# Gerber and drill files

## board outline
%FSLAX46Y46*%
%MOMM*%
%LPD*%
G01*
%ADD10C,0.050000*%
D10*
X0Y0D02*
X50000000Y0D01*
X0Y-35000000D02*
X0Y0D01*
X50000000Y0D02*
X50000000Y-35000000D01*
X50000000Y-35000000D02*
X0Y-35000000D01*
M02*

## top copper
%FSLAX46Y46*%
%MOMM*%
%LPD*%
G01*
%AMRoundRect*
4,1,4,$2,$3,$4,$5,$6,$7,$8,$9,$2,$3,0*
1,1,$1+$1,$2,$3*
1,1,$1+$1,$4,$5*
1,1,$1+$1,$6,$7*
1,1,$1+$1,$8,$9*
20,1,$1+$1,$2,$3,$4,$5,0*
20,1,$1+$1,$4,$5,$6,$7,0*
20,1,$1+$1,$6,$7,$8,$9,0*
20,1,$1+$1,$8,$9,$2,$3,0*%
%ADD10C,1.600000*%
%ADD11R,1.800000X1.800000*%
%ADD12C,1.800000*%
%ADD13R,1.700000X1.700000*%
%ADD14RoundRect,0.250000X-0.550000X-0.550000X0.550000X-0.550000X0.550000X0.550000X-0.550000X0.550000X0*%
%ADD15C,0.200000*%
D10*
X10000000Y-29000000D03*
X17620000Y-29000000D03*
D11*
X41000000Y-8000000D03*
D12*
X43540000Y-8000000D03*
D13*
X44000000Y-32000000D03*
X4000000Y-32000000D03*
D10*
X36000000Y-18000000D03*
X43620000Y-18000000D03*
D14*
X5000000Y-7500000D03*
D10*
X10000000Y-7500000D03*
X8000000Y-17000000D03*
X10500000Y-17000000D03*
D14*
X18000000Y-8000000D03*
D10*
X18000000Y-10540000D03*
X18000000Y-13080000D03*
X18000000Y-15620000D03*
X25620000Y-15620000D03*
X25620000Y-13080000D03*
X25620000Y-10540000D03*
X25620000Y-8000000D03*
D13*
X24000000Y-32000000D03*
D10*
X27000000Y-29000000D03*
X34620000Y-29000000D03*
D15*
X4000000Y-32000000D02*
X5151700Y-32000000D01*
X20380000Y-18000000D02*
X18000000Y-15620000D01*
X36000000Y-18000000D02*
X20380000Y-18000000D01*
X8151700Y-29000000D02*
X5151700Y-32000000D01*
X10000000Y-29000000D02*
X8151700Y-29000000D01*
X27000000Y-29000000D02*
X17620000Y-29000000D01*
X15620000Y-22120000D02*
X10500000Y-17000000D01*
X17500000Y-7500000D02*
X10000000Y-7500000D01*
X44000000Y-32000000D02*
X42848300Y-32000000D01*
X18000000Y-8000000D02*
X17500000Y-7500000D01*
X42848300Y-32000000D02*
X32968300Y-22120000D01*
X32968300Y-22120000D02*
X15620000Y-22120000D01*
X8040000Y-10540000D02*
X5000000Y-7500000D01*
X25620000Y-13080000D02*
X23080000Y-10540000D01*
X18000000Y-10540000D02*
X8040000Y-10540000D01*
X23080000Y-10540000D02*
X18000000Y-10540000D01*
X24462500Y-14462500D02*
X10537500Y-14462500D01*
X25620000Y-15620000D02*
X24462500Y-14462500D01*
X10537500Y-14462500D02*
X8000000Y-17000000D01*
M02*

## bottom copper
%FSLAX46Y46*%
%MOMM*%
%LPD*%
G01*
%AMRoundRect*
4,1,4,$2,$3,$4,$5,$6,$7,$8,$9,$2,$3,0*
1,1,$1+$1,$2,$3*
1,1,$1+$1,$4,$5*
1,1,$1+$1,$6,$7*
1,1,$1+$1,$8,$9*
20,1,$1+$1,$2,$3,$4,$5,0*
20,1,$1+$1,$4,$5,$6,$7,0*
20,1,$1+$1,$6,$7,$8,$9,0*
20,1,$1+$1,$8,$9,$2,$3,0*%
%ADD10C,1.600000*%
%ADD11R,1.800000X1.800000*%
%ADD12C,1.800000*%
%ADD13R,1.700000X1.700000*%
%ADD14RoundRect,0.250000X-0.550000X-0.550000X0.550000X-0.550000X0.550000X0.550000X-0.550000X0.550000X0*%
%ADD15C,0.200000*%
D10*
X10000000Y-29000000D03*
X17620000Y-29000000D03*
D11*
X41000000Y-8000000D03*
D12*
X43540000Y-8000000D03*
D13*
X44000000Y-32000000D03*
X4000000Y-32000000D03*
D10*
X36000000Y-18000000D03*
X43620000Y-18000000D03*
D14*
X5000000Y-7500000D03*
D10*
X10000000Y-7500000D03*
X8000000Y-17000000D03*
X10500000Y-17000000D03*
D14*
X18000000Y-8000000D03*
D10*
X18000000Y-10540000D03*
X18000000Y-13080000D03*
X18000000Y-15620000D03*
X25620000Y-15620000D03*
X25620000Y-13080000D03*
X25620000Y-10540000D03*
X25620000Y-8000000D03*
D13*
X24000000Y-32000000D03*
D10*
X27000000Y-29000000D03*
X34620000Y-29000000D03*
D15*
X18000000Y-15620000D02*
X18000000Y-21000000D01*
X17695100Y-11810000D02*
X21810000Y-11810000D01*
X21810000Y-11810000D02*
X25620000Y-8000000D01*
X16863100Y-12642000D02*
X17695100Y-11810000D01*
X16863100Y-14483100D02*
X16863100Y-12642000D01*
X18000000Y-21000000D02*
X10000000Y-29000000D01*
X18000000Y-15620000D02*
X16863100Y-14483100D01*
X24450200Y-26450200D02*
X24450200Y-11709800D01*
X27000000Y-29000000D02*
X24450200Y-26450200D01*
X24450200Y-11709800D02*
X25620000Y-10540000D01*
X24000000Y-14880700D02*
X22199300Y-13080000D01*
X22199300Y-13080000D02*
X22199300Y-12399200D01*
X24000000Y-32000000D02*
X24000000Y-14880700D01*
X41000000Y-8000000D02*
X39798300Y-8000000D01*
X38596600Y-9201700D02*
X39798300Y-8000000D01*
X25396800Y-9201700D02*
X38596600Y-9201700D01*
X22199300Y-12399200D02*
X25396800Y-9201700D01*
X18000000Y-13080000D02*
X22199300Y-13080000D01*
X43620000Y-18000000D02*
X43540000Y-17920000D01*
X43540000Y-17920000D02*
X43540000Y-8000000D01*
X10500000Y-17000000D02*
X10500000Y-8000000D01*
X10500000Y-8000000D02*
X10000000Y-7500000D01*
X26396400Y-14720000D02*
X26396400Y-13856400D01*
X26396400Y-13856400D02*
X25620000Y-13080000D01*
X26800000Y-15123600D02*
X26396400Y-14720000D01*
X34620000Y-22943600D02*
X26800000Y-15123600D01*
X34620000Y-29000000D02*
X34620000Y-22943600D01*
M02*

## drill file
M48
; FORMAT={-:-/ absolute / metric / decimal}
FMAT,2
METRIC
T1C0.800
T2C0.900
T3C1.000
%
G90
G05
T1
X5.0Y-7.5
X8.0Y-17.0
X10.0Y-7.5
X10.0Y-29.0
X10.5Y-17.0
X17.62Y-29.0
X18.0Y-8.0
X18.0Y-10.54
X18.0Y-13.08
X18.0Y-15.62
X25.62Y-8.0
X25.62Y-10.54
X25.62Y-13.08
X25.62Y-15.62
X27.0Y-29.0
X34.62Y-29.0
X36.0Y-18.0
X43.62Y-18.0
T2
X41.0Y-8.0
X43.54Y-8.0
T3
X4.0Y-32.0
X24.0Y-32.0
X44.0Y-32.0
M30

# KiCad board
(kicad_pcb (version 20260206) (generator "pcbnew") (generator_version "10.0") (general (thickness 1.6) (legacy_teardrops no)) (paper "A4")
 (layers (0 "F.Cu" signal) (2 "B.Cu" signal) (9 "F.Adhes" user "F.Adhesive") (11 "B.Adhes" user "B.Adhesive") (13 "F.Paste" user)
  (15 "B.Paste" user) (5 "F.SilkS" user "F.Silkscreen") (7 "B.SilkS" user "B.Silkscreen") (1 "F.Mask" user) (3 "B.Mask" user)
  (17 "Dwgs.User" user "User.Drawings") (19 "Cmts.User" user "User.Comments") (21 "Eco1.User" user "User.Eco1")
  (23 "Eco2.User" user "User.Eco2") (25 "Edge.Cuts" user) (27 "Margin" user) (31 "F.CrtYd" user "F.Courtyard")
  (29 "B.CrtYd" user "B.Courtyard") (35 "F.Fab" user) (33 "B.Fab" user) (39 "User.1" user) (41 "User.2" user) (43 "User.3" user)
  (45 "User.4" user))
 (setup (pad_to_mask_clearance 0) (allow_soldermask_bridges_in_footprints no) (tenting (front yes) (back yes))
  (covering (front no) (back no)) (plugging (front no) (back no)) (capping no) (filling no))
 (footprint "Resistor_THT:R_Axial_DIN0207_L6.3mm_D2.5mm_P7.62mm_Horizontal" (layer "F.Cu") (at 10 29)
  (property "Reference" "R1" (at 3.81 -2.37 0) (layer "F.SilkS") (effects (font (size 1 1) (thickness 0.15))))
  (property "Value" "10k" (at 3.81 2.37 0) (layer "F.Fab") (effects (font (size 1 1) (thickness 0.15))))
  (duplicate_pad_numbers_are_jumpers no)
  (pad "1" thru_hole circle (at 0 0) (size 1.6 1.6) (drill 0.8) (layers "*.Cu" "*.Mask") (remove_unused_layers no) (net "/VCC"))
  (pad "2" thru_hole circle (at 7.62 0) (size 1.6 1.6) (drill 0.8) (layers "*.Cu" "*.Mask") (remove_unused_layers no) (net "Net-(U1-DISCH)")))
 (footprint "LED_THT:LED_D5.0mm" (layer "F.Cu") (at 41 8)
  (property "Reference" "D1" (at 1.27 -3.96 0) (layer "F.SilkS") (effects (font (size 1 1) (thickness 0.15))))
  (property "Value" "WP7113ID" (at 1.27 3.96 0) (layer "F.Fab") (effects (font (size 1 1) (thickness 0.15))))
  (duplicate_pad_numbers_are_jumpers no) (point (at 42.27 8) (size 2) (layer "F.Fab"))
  (pad "1" thru_hole rect (at 0 0) (size 1.8 1.8) (drill 0.9) (layers "*.Cu" "*.Mask") (remove_unused_layers no) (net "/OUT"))
  (pad "2" thru_hole circle (at 2.54 0) (size 1.8 1.8) (drill 0.9) (layers "*.Cu" "*.Mask") (remove_unused_layers no) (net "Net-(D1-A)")))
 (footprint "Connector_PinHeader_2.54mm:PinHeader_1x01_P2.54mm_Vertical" (layer "F.Cu") (at 44 32)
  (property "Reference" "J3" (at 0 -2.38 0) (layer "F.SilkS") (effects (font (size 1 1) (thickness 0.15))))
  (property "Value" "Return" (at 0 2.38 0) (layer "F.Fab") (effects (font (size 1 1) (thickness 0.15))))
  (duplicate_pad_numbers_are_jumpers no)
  (pad "1" thru_hole rect (at 0 0) (size 1.7 1.7) (drill 1) (layers "*.Cu" "*.Mask") (remove_unused_layers no) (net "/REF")))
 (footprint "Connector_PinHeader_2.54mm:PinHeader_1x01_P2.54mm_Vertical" (layer "F.Cu") (at 4 32)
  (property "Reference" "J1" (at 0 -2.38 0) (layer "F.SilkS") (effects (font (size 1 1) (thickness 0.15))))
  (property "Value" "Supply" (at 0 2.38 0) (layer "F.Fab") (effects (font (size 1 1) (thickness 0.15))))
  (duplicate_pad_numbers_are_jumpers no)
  (pad "1" thru_hole rect (at 0 0) (size 1.7 1.7) (drill 1) (layers "*.Cu" "*.Mask") (remove_unused_layers no) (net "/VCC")))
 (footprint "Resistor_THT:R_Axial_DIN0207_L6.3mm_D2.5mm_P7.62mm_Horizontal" (layer "F.Cu") (at 36 18)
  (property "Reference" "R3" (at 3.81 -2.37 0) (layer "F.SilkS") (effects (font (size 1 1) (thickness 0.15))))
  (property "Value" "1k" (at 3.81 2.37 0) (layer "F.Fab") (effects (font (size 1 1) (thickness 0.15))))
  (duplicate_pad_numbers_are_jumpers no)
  (pad "1" thru_hole circle (at 0 0) (size 1.6 1.6) (drill 0.8) (layers "*.Cu" "*.Mask") (remove_unused_layers no) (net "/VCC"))
  (pad "2" thru_hole circle (at 7.62 0) (size 1.6 1.6) (drill 0.8) (layers "*.Cu" "*.Mask") (remove_unused_layers no) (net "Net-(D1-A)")))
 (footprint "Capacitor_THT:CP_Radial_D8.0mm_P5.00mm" (layer "F.Cu") (at 5 7.5)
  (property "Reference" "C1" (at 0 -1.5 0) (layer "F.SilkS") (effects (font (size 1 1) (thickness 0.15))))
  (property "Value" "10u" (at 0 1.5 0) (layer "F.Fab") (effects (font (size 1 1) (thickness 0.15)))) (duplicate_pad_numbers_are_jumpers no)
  (pad "1" thru_hole roundrect (at 0 0) (size 1.6 1.6) (drill 0.8) (layers "*.Cu" "*.Mask") (remove_unused_layers no)
   (roundrect_rratio 0.15625) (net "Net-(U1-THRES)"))
  (pad "2" thru_hole circle (at 5 0) (size 1.6 1.6) (drill 0.8) (layers "*.Cu" "*.Mask") (remove_unused_layers no) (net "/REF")))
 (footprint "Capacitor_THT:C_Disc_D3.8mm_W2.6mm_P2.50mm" (layer "F.Cu") (at 8 17)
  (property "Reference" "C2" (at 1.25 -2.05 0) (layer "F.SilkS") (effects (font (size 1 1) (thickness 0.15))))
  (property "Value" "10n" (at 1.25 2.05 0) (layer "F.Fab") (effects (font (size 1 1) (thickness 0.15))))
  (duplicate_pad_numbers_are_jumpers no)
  (pad "1" thru_hole circle (at 0 0) (size 1.6 1.6) (drill 0.8) (layers "*.Cu" "*.Mask") (remove_unused_layers no) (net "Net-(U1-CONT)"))
  (pad "2" thru_hole circle (at 2.5 0) (size 1.6 1.6) (drill 0.8) (layers "*.Cu" "*.Mask") (remove_unused_layers no) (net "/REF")))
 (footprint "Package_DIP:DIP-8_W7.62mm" (layer "F.Cu") (at 18 8)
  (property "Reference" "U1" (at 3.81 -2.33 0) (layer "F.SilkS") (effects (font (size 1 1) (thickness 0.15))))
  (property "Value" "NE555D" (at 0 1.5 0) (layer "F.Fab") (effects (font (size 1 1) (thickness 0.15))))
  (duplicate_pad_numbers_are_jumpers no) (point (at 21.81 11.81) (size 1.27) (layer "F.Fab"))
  (pad "1" thru_hole roundrect (at 0 0) (size 1.6 1.6) (drill 0.8) (layers "*.Cu" "*.Mask") (remove_unused_layers no)
   (roundrect_rratio 0.15625) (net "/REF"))
  (pad "2" thru_hole circle (at 0 2.54) (size 1.6 1.6) (drill 0.8) (layers "*.Cu" "*.Mask") (remove_unused_layers no) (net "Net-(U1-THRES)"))
  (pad "3" thru_hole circle (at 0 5.08) (size 1.6 1.6) (drill 0.8) (layers "*.Cu" "*.Mask") (remove_unused_layers no) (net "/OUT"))
  (pad "4" thru_hole circle (at 0 7.62) (size 1.6 1.6) (drill 0.8) (layers "*.Cu" "*.Mask") (remove_unused_layers no) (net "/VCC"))
  (pad "5" thru_hole circle (at 7.62 7.62) (size 1.6 1.6) (drill 0.8) (layers "*.Cu" "*.Mask") (remove_unused_layers no)
   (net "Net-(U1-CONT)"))
  (pad "6" thru_hole circle (at 7.62 5.08) (size 1.6 1.6) (drill 0.8) (layers "*.Cu" "*.Mask") (remove_unused_layers no)
   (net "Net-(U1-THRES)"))
  (pad "7" thru_hole circle (at 7.62 2.54) (size 1.6 1.6) (drill 0.8) (layers "*.Cu" "*.Mask") (remove_unused_layers no)
   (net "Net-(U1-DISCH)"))
  (pad "8" thru_hole circle (at 7.62 0) (size 1.6 1.6) (drill 0.8) (layers "*.Cu" "*.Mask") (remove_unused_layers no) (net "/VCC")))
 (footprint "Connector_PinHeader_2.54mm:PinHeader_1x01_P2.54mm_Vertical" (layer "F.Cu") (at 24 32)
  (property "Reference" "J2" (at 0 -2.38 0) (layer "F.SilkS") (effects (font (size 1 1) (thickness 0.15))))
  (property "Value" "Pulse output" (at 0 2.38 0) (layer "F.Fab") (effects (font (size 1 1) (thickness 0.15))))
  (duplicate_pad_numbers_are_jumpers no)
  (pad "1" thru_hole rect (at 0 0) (size 1.7 1.7) (drill 1) (layers "*.Cu" "*.Mask") (remove_unused_layers no) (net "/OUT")))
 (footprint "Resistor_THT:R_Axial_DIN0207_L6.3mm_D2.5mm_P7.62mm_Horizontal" (layer "F.Cu") (at 27 29)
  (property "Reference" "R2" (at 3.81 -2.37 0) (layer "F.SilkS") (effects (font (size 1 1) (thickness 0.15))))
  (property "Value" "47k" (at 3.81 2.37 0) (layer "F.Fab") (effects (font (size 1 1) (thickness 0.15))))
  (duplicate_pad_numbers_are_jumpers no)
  (pad "1" thru_hole circle (at 0 0) (size 1.6 1.6) (drill 0.8) (layers "*.Cu" "*.Mask") (remove_unused_layers no) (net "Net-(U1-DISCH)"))
  (pad "2" thru_hole circle (at 7.62 0) (size 1.6 1.6) (drill 0.8) (layers "*.Cu" "*.Mask") (remove_unused_layers no) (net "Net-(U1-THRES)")))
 (gr_line (start 0 0) (end 50 0) (stroke (width 0.05) (type default)) (layer "Edge.Cuts"))
 (gr_line (start 0 35) (end 0 0) (stroke (width 0.05) (type default)) (layer "Edge.Cuts"))
 (gr_line (start 50 0) (end 50 35) (stroke (width 0.05) (type default)) (layer "Edge.Cuts"))
 (gr_line (start 50 35) (end 0 35) (stroke (width 0.05) (type default)) (layer "Edge.Cuts"))
 (segment (start 4 32) (end 5.1517 32) (width 0.2) (layer "F.Cu") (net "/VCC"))
 (segment (start 20.38 18) (end 18 15.62) (width 0.2) (layer "F.Cu") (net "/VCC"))
 (segment (start 36 18) (end 20.38 18) (width 0.2) (layer "F.Cu") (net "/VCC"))
 (segment (start 8.1517 29) (end 5.1517 32) (width 0.2) (layer "F.Cu") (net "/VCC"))
 (segment (start 10 29) (end 8.1517 29) (width 0.2) (layer "F.Cu") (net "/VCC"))
 (segment (start 18 15.62) (end 18 21) (width 0.2) (layer "B.Cu") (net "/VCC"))
 (segment (start 17.6951 11.81) (end 21.81 11.81) (width 0.2) (layer "B.Cu") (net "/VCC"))
 (segment (start 21.81 11.81) (end 25.62 8) (width 0.2) (layer "B.Cu") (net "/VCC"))
 (segment (start 16.8631 12.642) (end 17.6951 11.81) (width 0.2) (layer "B.Cu") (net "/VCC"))
 (segment (start 16.8631 14.4831) (end 16.8631 12.642) (width 0.2) (layer "B.Cu") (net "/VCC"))
 (segment (start 18 21) (end 10 29) (width 0.2) (layer "B.Cu") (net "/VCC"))
 (segment (start 18 15.62) (end 16.8631 14.4831) (width 0.2) (layer "B.Cu") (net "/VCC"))
 (segment (start 27 29) (end 17.62 29) (width 0.2) (layer "F.Cu") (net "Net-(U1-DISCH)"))
 (segment (start 24.4502 26.4502) (end 24.4502 11.7098) (width 0.2) (layer "B.Cu") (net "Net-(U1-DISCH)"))
 (segment (start 27 29) (end 24.4502 26.4502) (width 0.2) (layer "B.Cu") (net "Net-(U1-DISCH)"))
 (segment (start 24.4502 11.7098) (end 25.62 10.54) (width 0.2) (layer "B.Cu") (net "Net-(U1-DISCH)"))
 (segment (start 24 14.8807) (end 22.1993 13.08) (width 0.2) (layer "B.Cu") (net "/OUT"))
 (segment (start 22.1993 13.08) (end 22.1993 12.3992) (width 0.2) (layer "B.Cu") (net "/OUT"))
 (segment (start 24 32) (end 24 14.8807) (width 0.2) (layer "B.Cu") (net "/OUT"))
 (segment (start 41 8) (end 39.7983 8) (width 0.2) (layer "B.Cu") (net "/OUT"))
 (segment (start 38.5966 9.2017) (end 39.7983 8) (width 0.2) (layer "B.Cu") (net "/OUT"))
 (segment (start 25.3968 9.2017) (end 38.5966 9.2017) (width 0.2) (layer "B.Cu") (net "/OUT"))
 (segment (start 22.1993 12.3992) (end 25.3968 9.2017) (width 0.2) (layer "B.Cu") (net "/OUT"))
 (segment (start 18 13.08) (end 22.1993 13.08) (width 0.2) (layer "B.Cu") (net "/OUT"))
 (segment (start 43.62 18) (end 43.54 17.92) (width 0.2) (layer "B.Cu") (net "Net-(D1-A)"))
 (segment (start 43.54 17.92) (end 43.54 8) (width 0.2) (layer "B.Cu") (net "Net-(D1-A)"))
 (segment (start 15.62 22.12) (end 10.5 17) (width 0.2) (layer "F.Cu") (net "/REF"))
 (segment (start 17.5 7.5) (end 10 7.5) (width 0.2) (layer "F.Cu") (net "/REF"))
 (segment (start 44 32) (end 42.8483 32) (width 0.2) (layer "F.Cu") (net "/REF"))
 (segment (start 18 8) (end 17.5 7.5) (width 0.2) (layer "F.Cu") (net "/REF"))
 (segment (start 42.8483 32) (end 32.9683 22.12) (width 0.2) (layer "F.Cu") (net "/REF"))
 (segment (start 32.9683 22.12) (end 15.62 22.12) (width 0.2) (layer "F.Cu") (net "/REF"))
 (segment (start 10.5 17) (end 10.5 8) (width 0.2) (layer "B.Cu") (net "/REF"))
 (segment (start 10.5 8) (end 10 7.5) (width 0.2) (layer "B.Cu") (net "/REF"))
 (segment (start 8.04 10.54) (end 5 7.5) (width 0.2) (layer "F.Cu") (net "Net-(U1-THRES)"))
 (segment (start 25.62 13.08) (end 23.08 10.54) (width 0.2) (layer "F.Cu") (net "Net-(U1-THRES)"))
 (segment (start 18 10.54) (end 8.04 10.54) (width 0.2) (layer "F.Cu") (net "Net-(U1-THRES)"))
 (segment (start 23.08 10.54) (end 18 10.54) (width 0.2) (layer "F.Cu") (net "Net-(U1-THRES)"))
 (segment (start 26.3964 14.72) (end 26.3964 13.8564) (width 0.2) (layer "B.Cu") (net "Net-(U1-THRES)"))
 (segment (start 26.3964 13.8564) (end 25.62 13.08) (width 0.2) (layer "B.Cu") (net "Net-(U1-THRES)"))
 (segment (start 26.8 15.1236) (end 26.3964 14.72) (width 0.2) (layer "B.Cu") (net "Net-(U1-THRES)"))
 (segment (start 34.62 22.9436) (end 26.8 15.1236) (width 0.2) (layer "B.Cu") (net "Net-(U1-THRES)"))
 (segment (start 34.62 29) (end 34.62 22.9436) (width 0.2) (layer "B.Cu") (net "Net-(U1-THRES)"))
 (segment (start 24.4625 14.4625) (end 10.5375 14.4625) (width 0.2) (layer "F.Cu") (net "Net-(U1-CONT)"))
 (segment (start 25.62 15.62) (end 24.4625 14.4625) (width 0.2) (layer "F.Cu") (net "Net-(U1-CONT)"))
 (segment (start 10.5375 14.4625) (end 8 17) (width 0.2) (layer "F.Cu") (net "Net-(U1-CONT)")))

